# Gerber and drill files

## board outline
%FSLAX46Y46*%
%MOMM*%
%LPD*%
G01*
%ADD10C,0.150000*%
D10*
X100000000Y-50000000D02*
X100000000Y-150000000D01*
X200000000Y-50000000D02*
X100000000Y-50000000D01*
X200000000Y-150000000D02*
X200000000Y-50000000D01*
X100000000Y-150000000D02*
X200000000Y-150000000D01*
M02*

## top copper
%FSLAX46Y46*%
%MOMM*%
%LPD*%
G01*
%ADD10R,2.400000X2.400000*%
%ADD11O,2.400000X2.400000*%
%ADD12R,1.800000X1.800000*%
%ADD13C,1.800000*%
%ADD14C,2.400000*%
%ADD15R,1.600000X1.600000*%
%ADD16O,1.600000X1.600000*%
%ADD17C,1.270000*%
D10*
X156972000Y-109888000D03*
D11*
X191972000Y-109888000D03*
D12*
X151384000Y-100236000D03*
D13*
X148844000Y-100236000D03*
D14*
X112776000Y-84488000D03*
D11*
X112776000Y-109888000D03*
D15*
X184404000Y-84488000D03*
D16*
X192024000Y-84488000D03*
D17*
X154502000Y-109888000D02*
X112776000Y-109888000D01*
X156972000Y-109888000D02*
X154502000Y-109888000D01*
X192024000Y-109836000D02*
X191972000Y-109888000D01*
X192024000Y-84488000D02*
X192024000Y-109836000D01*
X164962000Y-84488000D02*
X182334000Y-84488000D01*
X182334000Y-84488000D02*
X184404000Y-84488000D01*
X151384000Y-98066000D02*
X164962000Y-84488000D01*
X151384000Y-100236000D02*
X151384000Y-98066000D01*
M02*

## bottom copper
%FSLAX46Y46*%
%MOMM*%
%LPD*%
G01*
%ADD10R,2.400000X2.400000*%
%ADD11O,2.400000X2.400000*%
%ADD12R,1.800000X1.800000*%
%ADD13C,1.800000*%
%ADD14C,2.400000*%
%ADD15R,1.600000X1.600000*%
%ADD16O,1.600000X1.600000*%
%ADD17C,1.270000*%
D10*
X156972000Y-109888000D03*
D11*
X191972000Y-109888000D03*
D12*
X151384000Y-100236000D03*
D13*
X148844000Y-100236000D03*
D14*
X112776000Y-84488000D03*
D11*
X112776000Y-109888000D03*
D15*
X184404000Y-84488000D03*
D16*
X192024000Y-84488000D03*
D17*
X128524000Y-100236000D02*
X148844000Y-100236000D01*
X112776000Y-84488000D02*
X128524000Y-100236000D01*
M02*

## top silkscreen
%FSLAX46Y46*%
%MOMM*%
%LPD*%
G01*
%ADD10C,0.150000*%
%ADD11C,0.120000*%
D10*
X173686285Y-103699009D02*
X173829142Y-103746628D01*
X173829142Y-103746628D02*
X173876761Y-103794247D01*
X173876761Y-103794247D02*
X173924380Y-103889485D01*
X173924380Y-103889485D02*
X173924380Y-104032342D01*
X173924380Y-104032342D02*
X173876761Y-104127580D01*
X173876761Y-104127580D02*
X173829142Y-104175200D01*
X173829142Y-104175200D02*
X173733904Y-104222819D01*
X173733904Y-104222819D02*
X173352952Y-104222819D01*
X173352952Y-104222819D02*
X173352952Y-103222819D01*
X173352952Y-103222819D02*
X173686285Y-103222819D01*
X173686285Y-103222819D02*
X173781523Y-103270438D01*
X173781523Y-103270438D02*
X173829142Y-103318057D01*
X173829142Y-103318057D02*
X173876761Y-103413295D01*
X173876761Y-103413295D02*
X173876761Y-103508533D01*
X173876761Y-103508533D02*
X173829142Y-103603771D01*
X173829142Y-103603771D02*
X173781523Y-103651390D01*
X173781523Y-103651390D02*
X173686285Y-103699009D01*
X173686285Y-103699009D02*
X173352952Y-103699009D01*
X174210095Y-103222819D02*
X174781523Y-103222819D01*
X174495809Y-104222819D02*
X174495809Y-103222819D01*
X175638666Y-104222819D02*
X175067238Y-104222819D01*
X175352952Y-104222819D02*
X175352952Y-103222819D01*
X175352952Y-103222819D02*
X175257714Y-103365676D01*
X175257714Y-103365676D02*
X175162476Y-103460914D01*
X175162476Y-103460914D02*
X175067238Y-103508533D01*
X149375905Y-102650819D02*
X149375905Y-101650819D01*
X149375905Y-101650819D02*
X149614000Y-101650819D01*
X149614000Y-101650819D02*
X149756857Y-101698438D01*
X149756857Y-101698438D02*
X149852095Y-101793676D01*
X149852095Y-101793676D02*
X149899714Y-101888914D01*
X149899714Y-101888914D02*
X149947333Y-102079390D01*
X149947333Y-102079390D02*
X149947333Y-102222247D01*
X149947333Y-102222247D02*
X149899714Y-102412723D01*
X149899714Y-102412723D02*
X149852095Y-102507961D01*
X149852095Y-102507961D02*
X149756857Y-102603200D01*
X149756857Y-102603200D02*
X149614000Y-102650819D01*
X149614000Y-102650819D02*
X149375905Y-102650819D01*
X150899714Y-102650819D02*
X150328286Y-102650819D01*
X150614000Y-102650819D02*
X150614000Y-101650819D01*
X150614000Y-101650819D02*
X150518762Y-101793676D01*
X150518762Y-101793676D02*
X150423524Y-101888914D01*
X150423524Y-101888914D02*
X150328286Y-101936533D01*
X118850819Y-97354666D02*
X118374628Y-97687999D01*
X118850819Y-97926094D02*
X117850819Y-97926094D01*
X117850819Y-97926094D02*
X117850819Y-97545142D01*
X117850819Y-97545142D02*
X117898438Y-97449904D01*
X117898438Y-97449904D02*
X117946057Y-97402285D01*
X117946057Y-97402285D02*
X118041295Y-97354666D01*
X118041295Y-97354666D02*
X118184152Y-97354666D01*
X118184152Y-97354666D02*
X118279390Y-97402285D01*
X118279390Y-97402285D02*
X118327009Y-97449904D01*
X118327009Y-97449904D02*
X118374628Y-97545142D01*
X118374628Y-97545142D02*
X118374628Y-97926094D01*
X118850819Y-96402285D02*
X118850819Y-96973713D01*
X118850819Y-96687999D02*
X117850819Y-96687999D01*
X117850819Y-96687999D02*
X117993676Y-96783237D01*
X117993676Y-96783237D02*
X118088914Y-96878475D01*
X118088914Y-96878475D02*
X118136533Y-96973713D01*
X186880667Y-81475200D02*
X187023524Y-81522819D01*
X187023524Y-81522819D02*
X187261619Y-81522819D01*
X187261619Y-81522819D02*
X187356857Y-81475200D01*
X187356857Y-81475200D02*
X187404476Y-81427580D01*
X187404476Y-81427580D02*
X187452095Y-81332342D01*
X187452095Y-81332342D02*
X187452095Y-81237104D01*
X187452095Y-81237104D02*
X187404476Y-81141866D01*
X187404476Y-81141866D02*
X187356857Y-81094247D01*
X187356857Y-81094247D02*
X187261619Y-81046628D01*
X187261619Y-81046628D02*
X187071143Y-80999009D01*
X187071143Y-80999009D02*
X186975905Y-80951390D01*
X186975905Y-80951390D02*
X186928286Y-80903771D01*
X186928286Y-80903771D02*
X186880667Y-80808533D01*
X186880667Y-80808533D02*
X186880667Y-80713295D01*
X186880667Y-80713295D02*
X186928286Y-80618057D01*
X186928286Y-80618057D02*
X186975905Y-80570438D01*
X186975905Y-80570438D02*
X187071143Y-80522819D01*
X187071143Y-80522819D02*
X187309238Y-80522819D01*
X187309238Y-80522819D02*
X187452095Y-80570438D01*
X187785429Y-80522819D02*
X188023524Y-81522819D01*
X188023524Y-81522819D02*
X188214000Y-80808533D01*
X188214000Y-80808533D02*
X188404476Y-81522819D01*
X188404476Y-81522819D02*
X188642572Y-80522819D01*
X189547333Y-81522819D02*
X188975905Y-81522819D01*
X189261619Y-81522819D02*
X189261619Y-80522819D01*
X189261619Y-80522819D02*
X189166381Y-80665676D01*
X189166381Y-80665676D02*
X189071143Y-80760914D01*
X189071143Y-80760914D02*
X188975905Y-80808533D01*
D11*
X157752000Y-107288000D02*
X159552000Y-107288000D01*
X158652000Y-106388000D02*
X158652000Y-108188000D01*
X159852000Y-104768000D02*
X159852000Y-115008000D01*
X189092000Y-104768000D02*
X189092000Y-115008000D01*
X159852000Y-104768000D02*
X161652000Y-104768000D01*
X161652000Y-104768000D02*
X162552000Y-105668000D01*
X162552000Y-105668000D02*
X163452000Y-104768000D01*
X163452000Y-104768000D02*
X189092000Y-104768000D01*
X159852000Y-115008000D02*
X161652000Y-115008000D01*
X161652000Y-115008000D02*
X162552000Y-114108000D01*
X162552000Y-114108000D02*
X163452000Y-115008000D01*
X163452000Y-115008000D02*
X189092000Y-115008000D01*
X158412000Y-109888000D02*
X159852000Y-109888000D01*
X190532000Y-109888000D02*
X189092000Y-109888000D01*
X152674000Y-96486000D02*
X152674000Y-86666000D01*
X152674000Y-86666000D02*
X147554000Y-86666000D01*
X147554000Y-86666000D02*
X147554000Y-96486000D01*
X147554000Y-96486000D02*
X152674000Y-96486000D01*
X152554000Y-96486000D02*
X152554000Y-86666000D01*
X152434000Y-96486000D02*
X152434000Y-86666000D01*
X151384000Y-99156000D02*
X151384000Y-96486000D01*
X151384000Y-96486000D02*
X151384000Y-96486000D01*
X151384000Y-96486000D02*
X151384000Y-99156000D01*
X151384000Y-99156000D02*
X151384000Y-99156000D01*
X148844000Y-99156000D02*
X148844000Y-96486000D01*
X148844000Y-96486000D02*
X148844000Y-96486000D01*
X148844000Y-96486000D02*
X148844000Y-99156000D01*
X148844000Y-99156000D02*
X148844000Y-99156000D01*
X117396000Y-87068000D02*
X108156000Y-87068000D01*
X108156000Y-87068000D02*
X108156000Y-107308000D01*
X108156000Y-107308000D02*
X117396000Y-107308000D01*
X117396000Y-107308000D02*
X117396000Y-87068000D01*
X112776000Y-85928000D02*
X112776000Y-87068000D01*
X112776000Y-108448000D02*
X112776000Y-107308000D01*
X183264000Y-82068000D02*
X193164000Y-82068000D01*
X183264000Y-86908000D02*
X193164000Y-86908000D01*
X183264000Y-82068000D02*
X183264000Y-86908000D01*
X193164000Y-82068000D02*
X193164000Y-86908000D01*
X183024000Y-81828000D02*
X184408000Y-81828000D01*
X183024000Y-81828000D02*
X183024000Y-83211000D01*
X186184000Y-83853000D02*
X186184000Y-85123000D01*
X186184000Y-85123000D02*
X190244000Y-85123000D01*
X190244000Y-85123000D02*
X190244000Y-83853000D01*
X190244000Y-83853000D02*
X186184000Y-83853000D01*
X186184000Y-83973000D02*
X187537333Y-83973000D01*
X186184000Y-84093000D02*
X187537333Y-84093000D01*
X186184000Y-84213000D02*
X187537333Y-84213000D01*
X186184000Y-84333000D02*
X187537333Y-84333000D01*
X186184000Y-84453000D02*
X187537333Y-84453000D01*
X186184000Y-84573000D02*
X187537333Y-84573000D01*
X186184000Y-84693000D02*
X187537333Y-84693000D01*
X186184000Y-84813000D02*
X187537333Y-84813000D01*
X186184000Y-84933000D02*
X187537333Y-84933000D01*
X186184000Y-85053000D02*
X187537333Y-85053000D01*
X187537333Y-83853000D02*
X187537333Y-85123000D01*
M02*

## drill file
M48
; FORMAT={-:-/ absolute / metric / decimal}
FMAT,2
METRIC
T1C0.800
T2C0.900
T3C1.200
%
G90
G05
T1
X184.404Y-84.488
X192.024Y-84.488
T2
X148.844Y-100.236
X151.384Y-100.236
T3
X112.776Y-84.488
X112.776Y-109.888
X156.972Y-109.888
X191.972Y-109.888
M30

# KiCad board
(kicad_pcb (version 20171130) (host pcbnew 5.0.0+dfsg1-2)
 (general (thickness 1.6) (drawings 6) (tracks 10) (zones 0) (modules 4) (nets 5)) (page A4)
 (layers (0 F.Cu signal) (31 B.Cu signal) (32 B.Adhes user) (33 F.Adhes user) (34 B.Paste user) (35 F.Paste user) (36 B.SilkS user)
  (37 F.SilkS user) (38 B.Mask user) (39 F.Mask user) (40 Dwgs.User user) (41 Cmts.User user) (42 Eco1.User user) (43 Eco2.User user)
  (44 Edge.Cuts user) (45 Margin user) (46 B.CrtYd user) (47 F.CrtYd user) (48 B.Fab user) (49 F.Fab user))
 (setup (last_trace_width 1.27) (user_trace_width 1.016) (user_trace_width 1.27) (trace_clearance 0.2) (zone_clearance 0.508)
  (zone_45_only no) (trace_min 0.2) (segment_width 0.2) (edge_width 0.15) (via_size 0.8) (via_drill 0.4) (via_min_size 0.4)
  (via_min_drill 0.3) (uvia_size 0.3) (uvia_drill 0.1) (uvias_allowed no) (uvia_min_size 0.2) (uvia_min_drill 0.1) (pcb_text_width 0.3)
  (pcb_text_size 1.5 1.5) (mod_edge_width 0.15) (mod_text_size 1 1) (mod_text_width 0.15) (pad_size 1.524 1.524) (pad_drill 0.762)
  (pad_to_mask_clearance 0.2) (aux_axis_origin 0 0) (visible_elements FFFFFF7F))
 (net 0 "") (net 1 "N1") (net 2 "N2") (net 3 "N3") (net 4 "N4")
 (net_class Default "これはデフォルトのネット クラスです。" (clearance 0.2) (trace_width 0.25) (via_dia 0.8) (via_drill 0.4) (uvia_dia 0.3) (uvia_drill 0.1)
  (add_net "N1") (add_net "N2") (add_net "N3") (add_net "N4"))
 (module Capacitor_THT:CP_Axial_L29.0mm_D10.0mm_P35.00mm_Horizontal (layer F.Cu) (at 156.972 109.888)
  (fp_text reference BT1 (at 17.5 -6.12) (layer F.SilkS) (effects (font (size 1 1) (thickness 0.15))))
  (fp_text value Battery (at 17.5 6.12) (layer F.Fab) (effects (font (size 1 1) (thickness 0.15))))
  (fp_line (start 0.78 -2.6) (end 2.58 -2.6) (layer F.SilkS) (width 0.12))
  (fp_line (start 1.68 -3.5) (end 1.68 -1.7) (layer F.SilkS) (width 0.12))
  (fp_line (start 2.88 -5.12) (end 2.88 5.12) (layer F.SilkS) (width 0.12))
  (fp_line (start 32.12 -5.12) (end 32.12 5.12) (layer F.SilkS) (width 0.12))
  (fp_line (start 2.88 -5.12) (end 4.68 -5.12) (layer F.SilkS) (width 0.12))
  (fp_line (start 4.68 -5.12) (end 5.58 -4.22) (layer F.SilkS) (width 0.12))
  (fp_line (start 5.58 -4.22) (end 6.48 -5.12) (layer F.SilkS) (width 0.12))
  (fp_line (start 6.48 -5.12) (end 32.12 -5.12) (layer F.SilkS) (width 0.12))
  (fp_line (start 2.88 5.12) (end 4.68 5.12) (layer F.SilkS) (width 0.12))
  (fp_line (start 4.68 5.12) (end 5.58 4.22) (layer F.SilkS) (width 0.12))
  (fp_line (start 5.58 4.22) (end 6.48 5.12) (layer F.SilkS) (width 0.12))
  (fp_line (start 6.48 5.12) (end 32.12 5.12) (layer F.SilkS) (width 0.12))
  (fp_line (start 1.44 0) (end 2.88 0) (layer F.SilkS) (width 0.12))
  (fp_line (start 33.56 0) (end 32.12 0) (layer F.SilkS) (width 0.12))
  (pad 1 thru_hole rect (at 0 0) (size 2.4 2.4) (drill 1.2) (layers *.Cu *.Mask) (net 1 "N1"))
  (pad 2 thru_hole oval (at 35 0) (size 2.4 2.4) (drill 1.2) (layers *.Cu *.Mask) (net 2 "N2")))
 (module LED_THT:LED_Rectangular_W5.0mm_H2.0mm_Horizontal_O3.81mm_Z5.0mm (layer F.Cu) (at 151.384 100.236 180)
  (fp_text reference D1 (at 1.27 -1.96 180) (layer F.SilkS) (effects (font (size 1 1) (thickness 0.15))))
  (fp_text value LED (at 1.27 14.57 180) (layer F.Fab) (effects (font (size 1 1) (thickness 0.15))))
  (fp_line (start -1.29 3.75) (end -1.29 13.57) (layer F.SilkS) (width 0.12))
  (fp_line (start -1.29 13.57) (end 3.83 13.57) (layer F.SilkS) (width 0.12))
  (fp_line (start 3.83 13.57) (end 3.83 3.75) (layer F.SilkS) (width 0.12))
  (fp_line (start 3.83 3.75) (end -1.29 3.75) (layer F.SilkS) (width 0.12))
  (fp_line (start -1.17 3.75) (end -1.17 13.57) (layer F.SilkS) (width 0.12))
  (fp_line (start -1.05 3.75) (end -1.05 13.57) (layer F.SilkS) (width 0.12))
  (fp_line (start 0 1.08) (end 0 3.75) (layer F.SilkS) (width 0.12))
  (fp_line (start 0 3.75) (end 0 3.75) (layer F.SilkS) (width 0.12))
  (fp_line (start 0 3.75) (end 0 1.08) (layer F.SilkS) (width 0.12))
  (fp_line (start 0 1.08) (end 0 1.08) (layer F.SilkS) (width 0.12))
  (fp_line (start 2.54 1.08) (end 2.54 3.75) (layer F.SilkS) (width 0.12))
  (fp_line (start 2.54 3.75) (end 2.54 3.75) (layer F.SilkS) (width 0.12))
  (fp_line (start 2.54 3.75) (end 2.54 1.08) (layer F.SilkS) (width 0.12))
  (fp_line (start 2.54 1.08) (end 2.54 1.08) (layer F.SilkS) (width 0.12))
  (pad 1 thru_hole rect (at 0 0 180) (size 1.8 1.8) (drill 0.9) (layers *.Cu *.Mask) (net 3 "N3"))
  (pad 2 thru_hole circle (at 2.54 0 180) (size 1.8 1.8) (drill 0.9) (layers *.Cu *.Mask) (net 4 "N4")))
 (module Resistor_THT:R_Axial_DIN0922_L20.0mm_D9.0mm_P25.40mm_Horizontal (layer F.Cu) (at 112.776 84.488 270)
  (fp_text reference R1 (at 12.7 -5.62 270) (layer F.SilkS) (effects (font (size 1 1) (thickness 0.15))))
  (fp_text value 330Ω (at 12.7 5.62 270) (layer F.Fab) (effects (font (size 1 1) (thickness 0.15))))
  (fp_line (start 2.58 -4.62) (end 2.58 4.62) (layer F.SilkS) (width 0.12))
  (fp_line (start 2.58 4.62) (end 22.82 4.62) (layer F.SilkS) (width 0.12))
  (fp_line (start 22.82 4.62) (end 22.82 -4.62) (layer F.SilkS) (width 0.12))
  (fp_line (start 22.82 -4.62) (end 2.58 -4.62) (layer F.SilkS) (width 0.12))
  (fp_line (start 1.44 0) (end 2.58 0) (layer F.SilkS) (width 0.12))
  (fp_line (start 23.96 0) (end 22.82 0) (layer F.SilkS) (width 0.12))
  (pad 1 thru_hole circle (at 0 0 270) (size 2.4 2.4) (drill 1.2) (layers *.Cu *.Mask) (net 4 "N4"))
  (pad 2 thru_hole oval (at 25.4 0 270) (size 2.4 2.4) (drill 1.2) (layers *.Cu *.Mask) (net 1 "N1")))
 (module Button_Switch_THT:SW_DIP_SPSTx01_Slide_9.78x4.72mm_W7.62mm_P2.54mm (layer F.Cu) (at 184.404 84.488)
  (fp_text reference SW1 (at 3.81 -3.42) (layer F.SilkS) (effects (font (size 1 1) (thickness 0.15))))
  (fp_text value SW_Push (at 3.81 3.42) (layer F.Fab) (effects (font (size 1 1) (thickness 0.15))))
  (fp_line (start -1.14 -2.42) (end 8.76 -2.42) (layer F.SilkS) (width 0.12))
  (fp_line (start -1.14 2.42) (end 8.76 2.42) (layer F.SilkS) (width 0.12))
  (fp_line (start -1.14 -2.42) (end -1.14 2.42) (layer F.SilkS) (width 0.12))
  (fp_line (start 8.76 -2.42) (end 8.76 2.42) (layer F.SilkS) (width 0.12))
  (fp_line (start -1.38 -2.66) (end 0.004 -2.66) (layer F.SilkS) (width 0.12))
  (fp_line (start -1.38 -2.66) (end -1.38 -1.277) (layer F.SilkS) (width 0.12))
  (fp_line (start 1.78 -0.635) (end 1.78 0.635) (layer F.SilkS) (width 0.12))
  (fp_line (start 1.78 0.635) (end 5.84 0.635) (layer F.SilkS) (width 0.12))
  (fp_line (start 5.84 0.635) (end 5.84 -0.635) (layer F.SilkS) (width 0.12))
  (fp_line (start 5.84 -0.635) (end 1.78 -0.635) (layer F.SilkS) (width 0.12))
  (fp_line (start 1.78 -0.515) (end 3.133333 -0.515) (layer F.SilkS) (width 0.12))
  (fp_line (start 1.78 -0.395) (end 3.133333 -0.395) (layer F.SilkS) (width 0.12))
  (fp_line (start 1.78 -0.275) (end 3.133333 -0.275) (layer F.SilkS) (width 0.12))
  (fp_line (start 1.78 -0.155) (end 3.133333 -0.155) (layer F.SilkS) (width 0.12))
  (fp_line (start 1.78 -0.035) (end 3.133333 -0.035) (layer F.SilkS) (width 0.12))
  (fp_line (start 1.78 0.085) (end 3.133333 0.085) (layer F.SilkS) (width 0.12))
  (fp_line (start 1.78 0.205) (end 3.133333 0.205) (layer F.SilkS) (width 0.12))
  (fp_line (start 1.78 0.325) (end 3.133333 0.325) (layer F.SilkS) (width 0.12))
  (fp_line (start 1.78 0.445) (end 3.133333 0.445) (layer F.SilkS) (width 0.12))
  (fp_line (start 1.78 0.565) (end 3.133333 0.565) (layer F.SilkS) (width 0.12))
  (fp_line (start 3.133333 -0.635) (end 3.133333 0.635) (layer F.SilkS) (width 0.12))
  (pad 1 thru_hole rect (at 0 0) (size 1.6 1.6) (drill 0.8) (layers *.Cu *.Mask) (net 3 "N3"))
  (pad 2 thru_hole oval (at 7.62 0) (size 1.6 1.6) (drill 0.8) (layers *.Cu *.Mask) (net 2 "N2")))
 (gr_line (start 100 50) (end 100 150) (layer Edge.Cuts) (width 0.15))
 (gr_line (start 200 50) (end 100 50) (layer Edge.Cuts) (width 0.15))
 (gr_line (start 200 150) (end 200 50) (layer Edge.Cuts) (width 0.15))
 (gr_line (start 100 150) (end 200 150) (layer Edge.Cuts) (width 0.15))
 (segment (start 154.502 109.888) (end 112.776 109.888) (width 1.27) (layer F.Cu) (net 1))
 (segment (start 156.972 109.888) (end 154.502 109.888) (width 1.27) (layer F.Cu) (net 1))
 (segment (start 192.024 109.836) (end 191.972 109.888) (width 1.27) (layer F.Cu) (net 2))
 (segment (start 192.024 84.488) (end 192.024 109.836) (width 1.27) (layer F.Cu) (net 2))
 (segment (start 164.962 84.488) (end 182.334 84.488) (width 1.27) (layer F.Cu) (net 3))
 (segment (start 182.334 84.488) (end 184.404 84.488) (width 1.27) (layer F.Cu) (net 3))
 (segment (start 151.384 98.066) (end 164.962 84.488) (width 1.27) (layer F.Cu) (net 3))
 (segment (start 151.384 100.236) (end 151.384 98.066) (width 1.27) (layer F.Cu) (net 3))
 (segment (start 128.524 100.236) (end 148.844 100.236) (width 1.27) (layer B.Cu) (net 4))
 (segment (start 112.776 84.488) (end 128.524 100.236) (width 1.27) (layer B.Cu) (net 4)))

